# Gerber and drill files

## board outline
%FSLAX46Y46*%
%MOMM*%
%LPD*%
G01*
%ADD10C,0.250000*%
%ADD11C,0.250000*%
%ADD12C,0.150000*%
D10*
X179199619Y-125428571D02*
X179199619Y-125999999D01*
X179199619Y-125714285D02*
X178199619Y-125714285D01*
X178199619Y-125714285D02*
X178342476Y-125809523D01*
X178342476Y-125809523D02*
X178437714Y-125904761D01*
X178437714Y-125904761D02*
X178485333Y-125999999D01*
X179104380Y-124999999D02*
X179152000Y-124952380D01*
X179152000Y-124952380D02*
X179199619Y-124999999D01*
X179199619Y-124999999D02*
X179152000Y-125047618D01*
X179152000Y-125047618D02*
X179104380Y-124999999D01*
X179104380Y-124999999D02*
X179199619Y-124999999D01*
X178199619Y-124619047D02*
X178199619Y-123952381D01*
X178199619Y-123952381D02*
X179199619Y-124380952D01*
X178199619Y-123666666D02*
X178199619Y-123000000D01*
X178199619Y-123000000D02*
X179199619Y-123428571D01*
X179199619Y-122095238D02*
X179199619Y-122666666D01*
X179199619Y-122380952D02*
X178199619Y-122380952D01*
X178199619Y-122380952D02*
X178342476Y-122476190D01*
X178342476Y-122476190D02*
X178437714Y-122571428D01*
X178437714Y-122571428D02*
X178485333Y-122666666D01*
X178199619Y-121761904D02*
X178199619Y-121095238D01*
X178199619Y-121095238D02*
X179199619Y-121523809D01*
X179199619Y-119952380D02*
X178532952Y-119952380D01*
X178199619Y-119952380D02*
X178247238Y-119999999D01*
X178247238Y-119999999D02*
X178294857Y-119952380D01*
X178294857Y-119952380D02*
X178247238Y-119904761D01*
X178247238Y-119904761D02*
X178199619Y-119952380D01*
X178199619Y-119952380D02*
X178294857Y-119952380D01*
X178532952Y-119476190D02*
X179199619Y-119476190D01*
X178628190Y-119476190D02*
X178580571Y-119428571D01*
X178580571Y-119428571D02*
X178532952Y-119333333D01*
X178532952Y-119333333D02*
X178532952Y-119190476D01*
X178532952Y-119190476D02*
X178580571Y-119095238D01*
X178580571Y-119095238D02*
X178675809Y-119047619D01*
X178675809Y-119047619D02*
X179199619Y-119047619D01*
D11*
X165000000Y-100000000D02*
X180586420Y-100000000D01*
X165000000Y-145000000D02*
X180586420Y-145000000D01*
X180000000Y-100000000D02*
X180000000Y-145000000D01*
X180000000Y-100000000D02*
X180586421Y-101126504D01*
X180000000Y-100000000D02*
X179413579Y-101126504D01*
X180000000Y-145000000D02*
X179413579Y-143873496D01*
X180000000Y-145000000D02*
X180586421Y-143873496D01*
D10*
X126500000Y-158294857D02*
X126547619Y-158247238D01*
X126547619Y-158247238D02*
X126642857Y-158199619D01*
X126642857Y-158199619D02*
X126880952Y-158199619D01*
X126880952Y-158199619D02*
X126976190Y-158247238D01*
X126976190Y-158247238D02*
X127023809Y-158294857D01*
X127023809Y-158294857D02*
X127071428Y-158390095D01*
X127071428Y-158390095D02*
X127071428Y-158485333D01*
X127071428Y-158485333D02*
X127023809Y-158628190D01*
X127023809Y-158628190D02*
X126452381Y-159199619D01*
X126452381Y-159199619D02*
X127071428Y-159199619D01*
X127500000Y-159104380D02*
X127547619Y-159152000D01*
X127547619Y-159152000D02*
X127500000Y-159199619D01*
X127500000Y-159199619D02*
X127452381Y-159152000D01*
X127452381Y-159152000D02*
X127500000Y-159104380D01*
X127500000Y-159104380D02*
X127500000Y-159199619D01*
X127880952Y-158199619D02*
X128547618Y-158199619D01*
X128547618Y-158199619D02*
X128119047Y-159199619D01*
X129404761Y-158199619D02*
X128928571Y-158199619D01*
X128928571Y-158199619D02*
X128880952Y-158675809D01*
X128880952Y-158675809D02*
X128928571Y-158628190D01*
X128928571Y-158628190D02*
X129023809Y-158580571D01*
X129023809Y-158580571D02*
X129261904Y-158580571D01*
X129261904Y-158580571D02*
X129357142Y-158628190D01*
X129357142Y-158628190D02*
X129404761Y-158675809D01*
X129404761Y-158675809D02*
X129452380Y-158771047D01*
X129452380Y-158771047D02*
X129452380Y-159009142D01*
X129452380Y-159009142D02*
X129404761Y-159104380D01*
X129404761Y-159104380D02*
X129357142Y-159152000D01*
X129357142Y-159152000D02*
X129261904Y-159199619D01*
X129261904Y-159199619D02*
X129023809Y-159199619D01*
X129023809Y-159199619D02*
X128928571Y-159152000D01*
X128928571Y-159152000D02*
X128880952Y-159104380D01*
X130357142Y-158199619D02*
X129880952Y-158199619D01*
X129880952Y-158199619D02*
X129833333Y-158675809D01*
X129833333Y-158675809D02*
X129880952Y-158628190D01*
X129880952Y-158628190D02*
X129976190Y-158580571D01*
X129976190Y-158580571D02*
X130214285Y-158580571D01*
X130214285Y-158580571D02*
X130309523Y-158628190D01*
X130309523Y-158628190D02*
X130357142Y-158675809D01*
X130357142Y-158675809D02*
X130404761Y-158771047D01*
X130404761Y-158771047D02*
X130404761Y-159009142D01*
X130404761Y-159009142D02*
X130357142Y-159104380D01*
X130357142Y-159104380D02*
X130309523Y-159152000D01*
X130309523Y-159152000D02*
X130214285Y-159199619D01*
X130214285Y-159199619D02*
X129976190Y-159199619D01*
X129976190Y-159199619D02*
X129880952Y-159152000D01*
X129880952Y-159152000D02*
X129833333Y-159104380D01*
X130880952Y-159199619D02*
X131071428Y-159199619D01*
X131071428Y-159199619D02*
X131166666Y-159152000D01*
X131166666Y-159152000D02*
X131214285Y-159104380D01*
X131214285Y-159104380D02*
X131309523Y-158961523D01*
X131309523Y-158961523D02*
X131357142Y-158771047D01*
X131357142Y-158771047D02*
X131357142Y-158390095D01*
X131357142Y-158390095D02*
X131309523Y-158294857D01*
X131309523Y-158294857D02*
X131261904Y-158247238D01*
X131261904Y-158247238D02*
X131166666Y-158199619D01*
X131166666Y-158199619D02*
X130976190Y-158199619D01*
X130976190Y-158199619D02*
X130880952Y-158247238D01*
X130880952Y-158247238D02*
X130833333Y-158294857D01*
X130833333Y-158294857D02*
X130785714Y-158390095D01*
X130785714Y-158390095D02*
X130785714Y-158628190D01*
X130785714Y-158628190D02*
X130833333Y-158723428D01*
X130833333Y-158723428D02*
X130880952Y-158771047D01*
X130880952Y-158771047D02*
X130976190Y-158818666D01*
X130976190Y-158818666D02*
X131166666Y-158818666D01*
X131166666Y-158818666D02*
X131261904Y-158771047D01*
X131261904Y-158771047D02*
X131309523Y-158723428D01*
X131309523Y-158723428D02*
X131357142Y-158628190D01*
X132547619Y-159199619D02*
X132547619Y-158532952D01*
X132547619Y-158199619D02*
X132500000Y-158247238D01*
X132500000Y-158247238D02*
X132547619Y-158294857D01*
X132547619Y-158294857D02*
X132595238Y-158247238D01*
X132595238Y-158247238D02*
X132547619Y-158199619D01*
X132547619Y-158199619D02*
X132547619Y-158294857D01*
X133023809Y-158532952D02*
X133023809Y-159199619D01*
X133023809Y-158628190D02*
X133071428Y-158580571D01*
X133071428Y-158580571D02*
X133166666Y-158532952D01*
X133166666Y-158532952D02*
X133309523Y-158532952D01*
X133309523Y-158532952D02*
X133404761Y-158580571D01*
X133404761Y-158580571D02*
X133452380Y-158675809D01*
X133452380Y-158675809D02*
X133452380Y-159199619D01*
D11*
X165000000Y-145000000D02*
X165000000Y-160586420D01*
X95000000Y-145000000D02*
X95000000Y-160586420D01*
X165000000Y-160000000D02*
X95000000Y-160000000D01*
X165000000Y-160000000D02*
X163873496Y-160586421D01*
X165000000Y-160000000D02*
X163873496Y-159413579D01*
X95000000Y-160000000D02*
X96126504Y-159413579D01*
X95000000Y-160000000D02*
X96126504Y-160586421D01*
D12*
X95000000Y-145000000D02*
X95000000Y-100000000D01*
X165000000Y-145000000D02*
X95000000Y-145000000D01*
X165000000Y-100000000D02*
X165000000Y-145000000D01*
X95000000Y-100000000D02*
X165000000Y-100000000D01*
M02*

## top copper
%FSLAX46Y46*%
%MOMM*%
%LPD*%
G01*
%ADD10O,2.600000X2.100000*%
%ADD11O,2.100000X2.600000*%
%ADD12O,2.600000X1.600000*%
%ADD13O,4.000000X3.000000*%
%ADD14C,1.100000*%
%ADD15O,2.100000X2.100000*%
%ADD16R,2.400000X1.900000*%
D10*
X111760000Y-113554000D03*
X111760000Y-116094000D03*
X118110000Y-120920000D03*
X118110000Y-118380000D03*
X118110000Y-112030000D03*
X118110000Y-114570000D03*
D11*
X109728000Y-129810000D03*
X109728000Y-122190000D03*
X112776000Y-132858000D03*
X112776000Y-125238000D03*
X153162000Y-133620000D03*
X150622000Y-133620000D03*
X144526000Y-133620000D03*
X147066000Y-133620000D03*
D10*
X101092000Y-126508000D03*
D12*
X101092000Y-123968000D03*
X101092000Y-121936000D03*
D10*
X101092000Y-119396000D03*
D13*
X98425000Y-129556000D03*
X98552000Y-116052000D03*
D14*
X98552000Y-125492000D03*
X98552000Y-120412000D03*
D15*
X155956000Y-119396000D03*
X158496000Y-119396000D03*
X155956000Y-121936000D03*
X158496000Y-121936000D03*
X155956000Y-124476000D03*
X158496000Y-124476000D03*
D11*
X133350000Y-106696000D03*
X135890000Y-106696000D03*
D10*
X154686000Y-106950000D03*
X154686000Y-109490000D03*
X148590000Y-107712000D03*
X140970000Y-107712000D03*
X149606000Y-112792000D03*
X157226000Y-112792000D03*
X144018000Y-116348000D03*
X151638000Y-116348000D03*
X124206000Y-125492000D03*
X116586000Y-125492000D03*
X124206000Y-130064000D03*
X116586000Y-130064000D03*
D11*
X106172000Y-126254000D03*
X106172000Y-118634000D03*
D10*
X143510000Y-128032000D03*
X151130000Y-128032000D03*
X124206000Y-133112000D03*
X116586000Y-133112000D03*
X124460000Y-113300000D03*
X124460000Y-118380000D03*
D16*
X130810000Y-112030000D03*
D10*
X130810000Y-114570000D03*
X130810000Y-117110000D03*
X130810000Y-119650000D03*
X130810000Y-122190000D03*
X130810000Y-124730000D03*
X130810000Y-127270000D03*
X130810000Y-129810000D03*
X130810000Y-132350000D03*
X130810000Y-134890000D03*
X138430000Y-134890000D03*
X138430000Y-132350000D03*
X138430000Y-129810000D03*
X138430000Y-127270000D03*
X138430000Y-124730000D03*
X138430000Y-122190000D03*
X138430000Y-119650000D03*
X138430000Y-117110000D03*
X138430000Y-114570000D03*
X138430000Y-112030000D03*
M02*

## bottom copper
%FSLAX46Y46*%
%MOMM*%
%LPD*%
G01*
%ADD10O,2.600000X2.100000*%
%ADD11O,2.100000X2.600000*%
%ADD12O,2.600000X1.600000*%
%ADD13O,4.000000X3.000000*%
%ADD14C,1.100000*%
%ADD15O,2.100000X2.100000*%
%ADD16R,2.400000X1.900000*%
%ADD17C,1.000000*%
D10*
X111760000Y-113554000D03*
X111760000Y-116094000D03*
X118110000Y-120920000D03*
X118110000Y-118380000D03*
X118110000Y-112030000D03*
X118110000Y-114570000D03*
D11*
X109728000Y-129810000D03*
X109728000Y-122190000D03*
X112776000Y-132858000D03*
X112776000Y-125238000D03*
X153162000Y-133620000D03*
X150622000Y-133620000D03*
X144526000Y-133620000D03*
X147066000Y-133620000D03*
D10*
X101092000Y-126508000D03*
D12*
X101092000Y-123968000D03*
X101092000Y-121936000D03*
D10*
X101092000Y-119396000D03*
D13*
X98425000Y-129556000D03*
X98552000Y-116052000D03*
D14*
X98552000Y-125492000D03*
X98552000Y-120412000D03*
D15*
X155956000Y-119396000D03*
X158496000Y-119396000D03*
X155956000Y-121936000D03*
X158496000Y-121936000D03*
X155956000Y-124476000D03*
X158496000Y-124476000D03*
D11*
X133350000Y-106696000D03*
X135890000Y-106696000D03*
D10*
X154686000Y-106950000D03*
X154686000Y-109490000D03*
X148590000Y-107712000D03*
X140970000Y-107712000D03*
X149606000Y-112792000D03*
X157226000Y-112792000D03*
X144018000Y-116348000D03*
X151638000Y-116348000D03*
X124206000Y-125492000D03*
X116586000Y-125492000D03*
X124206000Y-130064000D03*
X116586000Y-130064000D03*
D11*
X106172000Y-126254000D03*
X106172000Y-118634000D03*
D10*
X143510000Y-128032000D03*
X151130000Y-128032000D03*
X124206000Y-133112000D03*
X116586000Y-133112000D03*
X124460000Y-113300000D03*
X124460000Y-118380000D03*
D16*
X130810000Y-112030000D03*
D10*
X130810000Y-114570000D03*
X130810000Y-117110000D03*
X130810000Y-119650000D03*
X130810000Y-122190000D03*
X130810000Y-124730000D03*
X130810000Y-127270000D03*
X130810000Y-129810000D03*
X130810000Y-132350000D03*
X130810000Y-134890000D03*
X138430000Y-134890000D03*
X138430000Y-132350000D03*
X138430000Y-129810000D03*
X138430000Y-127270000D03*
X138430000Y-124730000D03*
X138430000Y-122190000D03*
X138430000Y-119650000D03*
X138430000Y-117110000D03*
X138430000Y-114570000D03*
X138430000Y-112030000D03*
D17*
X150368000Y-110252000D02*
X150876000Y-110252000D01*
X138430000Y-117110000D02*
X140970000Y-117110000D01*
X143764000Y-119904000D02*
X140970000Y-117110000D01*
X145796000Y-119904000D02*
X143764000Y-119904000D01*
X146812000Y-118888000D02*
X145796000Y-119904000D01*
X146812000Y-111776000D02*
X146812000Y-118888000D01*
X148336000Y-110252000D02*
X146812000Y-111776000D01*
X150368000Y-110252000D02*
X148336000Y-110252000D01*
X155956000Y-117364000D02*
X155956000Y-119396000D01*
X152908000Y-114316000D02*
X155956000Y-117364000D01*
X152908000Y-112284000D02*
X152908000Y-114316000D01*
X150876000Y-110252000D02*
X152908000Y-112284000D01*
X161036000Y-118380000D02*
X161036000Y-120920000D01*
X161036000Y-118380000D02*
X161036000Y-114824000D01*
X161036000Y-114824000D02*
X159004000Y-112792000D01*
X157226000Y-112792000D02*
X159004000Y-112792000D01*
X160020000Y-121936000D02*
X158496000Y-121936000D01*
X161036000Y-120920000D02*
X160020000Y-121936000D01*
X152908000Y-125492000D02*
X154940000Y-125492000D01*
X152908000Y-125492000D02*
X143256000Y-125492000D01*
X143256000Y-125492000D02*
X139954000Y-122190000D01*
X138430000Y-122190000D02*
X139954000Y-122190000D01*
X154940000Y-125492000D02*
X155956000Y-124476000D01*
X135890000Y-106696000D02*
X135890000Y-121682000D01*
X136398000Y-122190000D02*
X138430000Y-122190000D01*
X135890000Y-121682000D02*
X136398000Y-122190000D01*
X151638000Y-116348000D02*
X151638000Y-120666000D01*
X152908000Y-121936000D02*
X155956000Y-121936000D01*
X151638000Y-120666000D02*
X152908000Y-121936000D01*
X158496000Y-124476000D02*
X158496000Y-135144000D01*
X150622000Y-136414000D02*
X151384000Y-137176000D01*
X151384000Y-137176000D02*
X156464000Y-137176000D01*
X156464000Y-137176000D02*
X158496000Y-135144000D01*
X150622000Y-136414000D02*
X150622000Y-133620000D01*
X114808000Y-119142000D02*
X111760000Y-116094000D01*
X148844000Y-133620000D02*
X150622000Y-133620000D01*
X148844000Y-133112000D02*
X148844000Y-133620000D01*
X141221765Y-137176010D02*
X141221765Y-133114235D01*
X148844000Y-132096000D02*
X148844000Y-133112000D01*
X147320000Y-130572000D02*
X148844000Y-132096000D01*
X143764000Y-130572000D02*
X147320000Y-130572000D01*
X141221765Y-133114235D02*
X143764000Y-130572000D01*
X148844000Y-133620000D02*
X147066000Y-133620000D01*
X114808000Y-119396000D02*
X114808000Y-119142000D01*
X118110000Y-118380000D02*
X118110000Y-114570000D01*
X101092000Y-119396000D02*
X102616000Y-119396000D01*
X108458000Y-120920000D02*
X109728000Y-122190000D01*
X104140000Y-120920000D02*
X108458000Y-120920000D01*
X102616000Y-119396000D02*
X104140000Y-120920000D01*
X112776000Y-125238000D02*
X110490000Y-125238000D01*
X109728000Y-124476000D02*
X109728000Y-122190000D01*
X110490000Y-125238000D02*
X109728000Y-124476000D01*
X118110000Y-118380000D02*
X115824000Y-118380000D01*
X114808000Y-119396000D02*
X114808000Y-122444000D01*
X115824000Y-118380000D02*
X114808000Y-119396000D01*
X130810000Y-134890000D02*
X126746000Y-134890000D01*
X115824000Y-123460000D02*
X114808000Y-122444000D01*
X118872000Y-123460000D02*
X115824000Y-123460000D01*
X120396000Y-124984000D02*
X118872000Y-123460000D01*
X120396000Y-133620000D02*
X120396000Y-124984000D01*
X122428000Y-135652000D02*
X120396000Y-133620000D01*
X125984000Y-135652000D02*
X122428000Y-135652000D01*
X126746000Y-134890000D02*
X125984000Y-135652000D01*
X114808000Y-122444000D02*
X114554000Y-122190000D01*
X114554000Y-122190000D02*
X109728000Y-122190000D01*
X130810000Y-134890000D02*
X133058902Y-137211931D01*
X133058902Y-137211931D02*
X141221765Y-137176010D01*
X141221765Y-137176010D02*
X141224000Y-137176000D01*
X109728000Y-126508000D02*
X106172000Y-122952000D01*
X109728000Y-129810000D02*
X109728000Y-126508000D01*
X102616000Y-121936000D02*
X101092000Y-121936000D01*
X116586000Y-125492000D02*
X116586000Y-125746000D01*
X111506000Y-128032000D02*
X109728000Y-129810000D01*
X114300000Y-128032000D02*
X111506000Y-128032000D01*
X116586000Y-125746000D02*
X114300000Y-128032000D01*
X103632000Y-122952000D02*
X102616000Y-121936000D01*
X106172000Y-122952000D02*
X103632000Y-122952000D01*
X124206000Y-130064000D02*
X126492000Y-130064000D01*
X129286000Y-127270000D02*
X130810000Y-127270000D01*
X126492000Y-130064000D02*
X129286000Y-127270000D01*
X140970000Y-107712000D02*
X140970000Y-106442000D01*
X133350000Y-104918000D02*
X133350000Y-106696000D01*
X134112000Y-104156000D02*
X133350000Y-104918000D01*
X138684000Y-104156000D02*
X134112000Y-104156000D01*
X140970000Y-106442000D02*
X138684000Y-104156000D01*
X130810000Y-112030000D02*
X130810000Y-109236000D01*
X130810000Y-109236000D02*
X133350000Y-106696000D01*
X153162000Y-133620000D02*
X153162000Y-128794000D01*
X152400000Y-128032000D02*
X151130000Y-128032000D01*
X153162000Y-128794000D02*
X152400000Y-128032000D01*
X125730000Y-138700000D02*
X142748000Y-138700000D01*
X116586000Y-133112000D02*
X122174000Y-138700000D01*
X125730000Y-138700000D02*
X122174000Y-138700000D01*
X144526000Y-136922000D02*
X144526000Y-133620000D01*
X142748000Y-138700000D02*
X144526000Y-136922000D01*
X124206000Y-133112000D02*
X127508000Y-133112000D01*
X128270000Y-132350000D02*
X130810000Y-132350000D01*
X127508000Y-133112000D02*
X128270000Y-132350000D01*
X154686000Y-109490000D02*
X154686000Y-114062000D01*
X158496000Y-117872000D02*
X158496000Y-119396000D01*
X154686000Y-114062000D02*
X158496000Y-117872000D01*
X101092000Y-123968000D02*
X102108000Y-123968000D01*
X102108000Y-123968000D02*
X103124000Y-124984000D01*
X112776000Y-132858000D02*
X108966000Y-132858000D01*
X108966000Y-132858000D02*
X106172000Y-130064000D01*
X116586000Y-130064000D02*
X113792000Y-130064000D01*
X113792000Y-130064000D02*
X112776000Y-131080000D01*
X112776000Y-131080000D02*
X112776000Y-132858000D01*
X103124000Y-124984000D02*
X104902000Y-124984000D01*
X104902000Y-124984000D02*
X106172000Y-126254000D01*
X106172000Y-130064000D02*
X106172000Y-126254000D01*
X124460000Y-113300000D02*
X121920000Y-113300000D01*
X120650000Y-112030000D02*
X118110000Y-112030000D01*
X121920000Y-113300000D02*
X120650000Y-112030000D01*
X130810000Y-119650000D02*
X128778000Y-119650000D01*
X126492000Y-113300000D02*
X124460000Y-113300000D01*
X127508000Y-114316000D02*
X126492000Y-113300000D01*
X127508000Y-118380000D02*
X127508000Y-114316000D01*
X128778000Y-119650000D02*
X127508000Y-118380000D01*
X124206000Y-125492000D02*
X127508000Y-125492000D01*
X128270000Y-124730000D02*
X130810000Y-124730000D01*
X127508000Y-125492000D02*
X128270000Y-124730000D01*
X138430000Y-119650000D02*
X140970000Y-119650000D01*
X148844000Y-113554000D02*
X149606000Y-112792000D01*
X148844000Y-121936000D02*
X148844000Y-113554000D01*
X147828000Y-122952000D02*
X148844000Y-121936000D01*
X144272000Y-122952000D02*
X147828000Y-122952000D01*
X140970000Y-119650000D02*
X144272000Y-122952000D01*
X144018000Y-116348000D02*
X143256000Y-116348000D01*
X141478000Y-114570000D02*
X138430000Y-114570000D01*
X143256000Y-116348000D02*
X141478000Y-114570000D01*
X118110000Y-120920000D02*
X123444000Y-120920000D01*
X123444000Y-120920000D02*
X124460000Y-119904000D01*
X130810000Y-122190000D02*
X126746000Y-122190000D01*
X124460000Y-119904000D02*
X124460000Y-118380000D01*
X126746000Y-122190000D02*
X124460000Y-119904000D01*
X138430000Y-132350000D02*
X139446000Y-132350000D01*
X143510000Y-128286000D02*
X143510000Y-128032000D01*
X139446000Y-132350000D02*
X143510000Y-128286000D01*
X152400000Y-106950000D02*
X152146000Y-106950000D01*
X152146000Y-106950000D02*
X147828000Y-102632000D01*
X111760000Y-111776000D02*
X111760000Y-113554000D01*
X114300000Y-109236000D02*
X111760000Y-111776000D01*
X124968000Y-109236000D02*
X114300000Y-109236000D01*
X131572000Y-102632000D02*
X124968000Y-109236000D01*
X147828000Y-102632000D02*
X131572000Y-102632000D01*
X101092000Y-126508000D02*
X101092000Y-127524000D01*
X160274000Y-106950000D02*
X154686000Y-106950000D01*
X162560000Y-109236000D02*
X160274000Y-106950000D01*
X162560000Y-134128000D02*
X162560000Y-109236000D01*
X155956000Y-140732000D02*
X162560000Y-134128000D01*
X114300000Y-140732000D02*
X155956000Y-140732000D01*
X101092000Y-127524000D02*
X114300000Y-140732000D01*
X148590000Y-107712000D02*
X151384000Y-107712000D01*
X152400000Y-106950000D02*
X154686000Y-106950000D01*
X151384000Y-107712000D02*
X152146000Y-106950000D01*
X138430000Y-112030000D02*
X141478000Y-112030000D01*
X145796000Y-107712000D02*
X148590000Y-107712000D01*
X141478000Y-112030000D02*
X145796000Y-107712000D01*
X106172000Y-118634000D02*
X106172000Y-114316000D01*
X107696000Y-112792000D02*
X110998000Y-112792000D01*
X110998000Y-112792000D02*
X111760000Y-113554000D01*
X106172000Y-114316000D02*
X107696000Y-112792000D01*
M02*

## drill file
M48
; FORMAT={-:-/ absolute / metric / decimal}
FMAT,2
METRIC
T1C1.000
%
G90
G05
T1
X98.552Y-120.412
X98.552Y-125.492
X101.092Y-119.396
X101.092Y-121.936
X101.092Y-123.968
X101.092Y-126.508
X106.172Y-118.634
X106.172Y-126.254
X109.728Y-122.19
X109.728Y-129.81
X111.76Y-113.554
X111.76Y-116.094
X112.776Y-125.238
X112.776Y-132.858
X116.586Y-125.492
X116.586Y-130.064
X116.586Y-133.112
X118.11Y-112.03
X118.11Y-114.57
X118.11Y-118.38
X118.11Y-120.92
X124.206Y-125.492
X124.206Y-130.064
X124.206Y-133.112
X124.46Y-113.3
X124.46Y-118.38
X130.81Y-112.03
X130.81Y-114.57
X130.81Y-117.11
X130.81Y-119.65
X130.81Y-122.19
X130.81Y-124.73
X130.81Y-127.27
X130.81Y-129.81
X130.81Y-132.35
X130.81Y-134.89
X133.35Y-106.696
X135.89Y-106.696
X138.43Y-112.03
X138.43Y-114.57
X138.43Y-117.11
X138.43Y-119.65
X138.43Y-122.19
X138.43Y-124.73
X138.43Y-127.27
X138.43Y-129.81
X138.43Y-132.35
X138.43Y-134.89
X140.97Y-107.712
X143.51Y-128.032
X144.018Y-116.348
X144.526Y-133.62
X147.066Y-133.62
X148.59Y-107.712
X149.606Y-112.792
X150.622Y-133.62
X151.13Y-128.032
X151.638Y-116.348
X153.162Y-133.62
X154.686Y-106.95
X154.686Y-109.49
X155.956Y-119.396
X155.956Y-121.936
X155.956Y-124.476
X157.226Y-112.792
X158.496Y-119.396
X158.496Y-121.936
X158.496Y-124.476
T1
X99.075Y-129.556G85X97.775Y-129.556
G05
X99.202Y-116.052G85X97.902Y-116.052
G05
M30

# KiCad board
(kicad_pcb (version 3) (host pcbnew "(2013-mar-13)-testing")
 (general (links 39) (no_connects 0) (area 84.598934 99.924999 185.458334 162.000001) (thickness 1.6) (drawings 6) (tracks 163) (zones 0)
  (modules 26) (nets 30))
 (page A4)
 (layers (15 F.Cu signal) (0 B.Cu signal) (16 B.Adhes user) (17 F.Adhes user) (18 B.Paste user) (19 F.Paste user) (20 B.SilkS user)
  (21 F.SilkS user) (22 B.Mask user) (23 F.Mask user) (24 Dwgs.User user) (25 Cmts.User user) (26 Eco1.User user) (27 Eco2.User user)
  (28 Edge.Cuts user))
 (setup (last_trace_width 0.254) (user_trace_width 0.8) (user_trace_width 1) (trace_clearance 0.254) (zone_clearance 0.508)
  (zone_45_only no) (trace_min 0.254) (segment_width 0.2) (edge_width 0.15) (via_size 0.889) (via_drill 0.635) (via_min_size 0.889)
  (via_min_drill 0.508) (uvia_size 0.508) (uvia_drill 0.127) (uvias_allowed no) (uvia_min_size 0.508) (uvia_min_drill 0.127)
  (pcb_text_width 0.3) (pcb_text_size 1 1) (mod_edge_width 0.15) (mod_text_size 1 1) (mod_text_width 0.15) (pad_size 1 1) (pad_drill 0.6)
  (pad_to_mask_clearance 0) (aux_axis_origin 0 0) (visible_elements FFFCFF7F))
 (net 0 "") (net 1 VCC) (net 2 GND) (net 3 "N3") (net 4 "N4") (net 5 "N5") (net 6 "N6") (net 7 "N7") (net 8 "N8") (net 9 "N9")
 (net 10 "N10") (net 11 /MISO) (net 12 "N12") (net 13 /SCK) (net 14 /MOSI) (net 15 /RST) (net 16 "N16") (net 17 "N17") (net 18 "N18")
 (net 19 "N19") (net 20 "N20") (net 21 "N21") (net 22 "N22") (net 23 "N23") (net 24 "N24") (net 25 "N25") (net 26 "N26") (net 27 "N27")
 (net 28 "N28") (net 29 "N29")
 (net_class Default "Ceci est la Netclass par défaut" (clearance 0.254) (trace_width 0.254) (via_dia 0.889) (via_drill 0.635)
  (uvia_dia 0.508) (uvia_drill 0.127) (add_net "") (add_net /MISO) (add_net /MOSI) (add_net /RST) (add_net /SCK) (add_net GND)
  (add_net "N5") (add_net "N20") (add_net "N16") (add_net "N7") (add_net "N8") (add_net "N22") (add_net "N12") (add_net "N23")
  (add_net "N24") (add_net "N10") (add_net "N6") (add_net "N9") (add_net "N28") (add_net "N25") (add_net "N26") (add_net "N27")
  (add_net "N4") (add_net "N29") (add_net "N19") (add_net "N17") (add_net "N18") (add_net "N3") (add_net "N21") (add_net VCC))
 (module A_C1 (layer F.Cu) (at 111.76 114.824 270)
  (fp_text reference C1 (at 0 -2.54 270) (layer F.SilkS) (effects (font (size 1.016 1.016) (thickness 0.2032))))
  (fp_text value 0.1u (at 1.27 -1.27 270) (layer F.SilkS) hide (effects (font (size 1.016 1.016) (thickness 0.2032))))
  (pad 1 thru_hole oval (at -1.27 0 270) (size 2.1 2.6) (drill 1) (layers *.Cu *.Mask F.SilkS) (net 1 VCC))
  (pad 2 thru_hole oval (at 1.27 0 270) (size 2.1 2.6) (drill 1) (layers *.Cu *.Mask F.SilkS) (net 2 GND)))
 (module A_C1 (layer F.Cu) (at 118.11 119.65 90)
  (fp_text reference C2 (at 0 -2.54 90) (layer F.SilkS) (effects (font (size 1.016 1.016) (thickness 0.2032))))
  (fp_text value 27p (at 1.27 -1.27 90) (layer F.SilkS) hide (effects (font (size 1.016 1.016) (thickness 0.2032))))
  (pad 1 thru_hole oval (at -1.27 0 90) (size 2.1 2.6) (drill 1) (layers *.Cu *.Mask F.SilkS) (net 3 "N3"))
  (pad 2 thru_hole oval (at 1.27 0 90) (size 2.1 2.6) (drill 1) (layers *.Cu *.Mask F.SilkS) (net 2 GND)))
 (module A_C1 (layer F.Cu) (at 118.11 113.3 270)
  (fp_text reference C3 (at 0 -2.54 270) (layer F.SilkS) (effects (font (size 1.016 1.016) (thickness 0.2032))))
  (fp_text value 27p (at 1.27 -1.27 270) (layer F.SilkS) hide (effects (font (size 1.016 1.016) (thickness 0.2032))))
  (pad 1 thru_hole oval (at -1.27 0 270) (size 2.1 2.6) (drill 1) (layers *.Cu *.Mask F.SilkS) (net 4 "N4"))
  (pad 2 thru_hole oval (at 1.27 0 270) (size 2.1 2.6) (drill 1) (layers *.Cu *.Mask F.SilkS) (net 2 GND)))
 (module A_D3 (layer F.Cu) (at 109.728 126 270)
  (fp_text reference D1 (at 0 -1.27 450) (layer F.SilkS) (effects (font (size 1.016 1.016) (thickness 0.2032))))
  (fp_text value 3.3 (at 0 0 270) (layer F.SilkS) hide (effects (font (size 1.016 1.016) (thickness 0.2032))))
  (pad 2 thru_hole oval (at 3.81 0 270) (size 2.6 2.1) (drill 1) (layers *.Cu *.Mask F.SilkS) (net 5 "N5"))
  (pad 1 thru_hole oval (at -3.81 0 270) (size 2.6 2.1) (drill 1) (layers *.Cu *.Mask F.SilkS) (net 2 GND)))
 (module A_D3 (layer F.Cu) (at 112.776 129.048 270)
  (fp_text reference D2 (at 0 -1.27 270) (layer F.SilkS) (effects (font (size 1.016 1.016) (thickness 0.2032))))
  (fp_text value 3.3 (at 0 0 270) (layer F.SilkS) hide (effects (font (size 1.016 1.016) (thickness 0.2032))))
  (pad 2 thru_hole oval (at 3.81 0 270) (size 2.6 2.1) (drill 1) (layers *.Cu *.Mask F.SilkS) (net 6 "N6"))
  (pad 1 thru_hole oval (at -3.81 0 270) (size 2.6 2.1) (drill 1) (layers *.Cu *.Mask F.SilkS) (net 2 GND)))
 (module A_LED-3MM (layer F.Cu) (at 151.892 133.62 180)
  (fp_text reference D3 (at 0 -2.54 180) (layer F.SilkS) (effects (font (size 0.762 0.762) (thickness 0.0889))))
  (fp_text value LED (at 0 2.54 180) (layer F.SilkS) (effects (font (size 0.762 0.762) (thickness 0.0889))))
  (pad 1 thru_hole oval (at -1.27 0 180) (size 2.1 2.6) (drill 1) (layers *.Cu *.Mask F.SilkS) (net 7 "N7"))
  (pad 2 thru_hole oval (at 1.27 0 180) (size 2.1 2.6) (drill 1) (layers *.Cu *.Mask F.SilkS) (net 2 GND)))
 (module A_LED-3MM (layer F.Cu) (at 145.796 133.62)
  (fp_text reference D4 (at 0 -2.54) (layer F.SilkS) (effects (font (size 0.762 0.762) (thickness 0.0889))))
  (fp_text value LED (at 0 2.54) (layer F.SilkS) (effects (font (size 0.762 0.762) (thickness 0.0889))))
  (pad 1 thru_hole oval (at -1.27 0) (size 2.1 2.6) (drill 1) (layers *.Cu *.Mask F.SilkS) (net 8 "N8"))
  (pad 2 thru_hole oval (at 1.27 0) (size 2.1 2.6) (drill 1) (layers *.Cu *.Mask F.SilkS) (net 2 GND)))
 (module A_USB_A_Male (layer F.Cu) (at 101.092 122.952 180)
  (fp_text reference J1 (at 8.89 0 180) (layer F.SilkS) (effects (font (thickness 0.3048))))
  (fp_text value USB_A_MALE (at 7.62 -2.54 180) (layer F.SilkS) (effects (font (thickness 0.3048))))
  (pad 1 thru_hole oval (at 0 -3.556 180) (size 2.6 2.1) (drill 1) (layers *.Cu *.Mask F.SilkS) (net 1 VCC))
  (pad 2 thru_hole oval (at 0 -1.016 180) (size 2.6 1.6) (drill 1) (layers *.Cu *.Mask F.SilkS) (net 6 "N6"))
  (pad 3 thru_hole oval (at 0 1.016 180) (size 2.6 1.6) (drill 1) (layers *.Cu *.Mask F.SilkS) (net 5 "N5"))
  (pad 4 thru_hole oval (at 0 3.556 180) (size 2.6 2.1) (drill 1) (layers *.Cu *.Mask F.SilkS) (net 2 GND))
  (pad 6 thru_hole oval (at 2.667 -6.604 180) (size 4 3) (drill oval 2.3 1) (layers *.Cu *.Mask F.SilkS) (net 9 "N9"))
  (pad 5 thru_hole oval (at 2.54 6.9 180) (size 4 3) (drill oval 2.3 1) (layers *.Cu *.Mask F.SilkS) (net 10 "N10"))
  (pad "" thru_hole circle (at 2.54 -2.54 180) (size 1.1 1.1) (drill 1) (layers *.Cu *.Mask F.SilkS))
  (pad "" thru_hole circle (at 2.54 2.54 180) (size 1.1 1.1) (drill 1) (layers *.Cu *.Mask F.SilkS)))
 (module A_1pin (layer F.Cu) (at 155.956 119.396)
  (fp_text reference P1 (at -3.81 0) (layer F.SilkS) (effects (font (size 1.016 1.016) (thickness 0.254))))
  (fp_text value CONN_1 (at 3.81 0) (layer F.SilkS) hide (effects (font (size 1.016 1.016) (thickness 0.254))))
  (pad 1 thru_hole oval (at 0 0) (size 2.1 2.1) (drill 1) (layers *.Cu *.Mask F.SilkS) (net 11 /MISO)))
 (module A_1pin (layer F.Cu) (at 158.496 119.396)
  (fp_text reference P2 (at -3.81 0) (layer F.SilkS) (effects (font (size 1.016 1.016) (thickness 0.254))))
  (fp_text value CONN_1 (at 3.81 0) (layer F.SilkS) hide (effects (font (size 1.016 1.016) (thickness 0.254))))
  (pad 1 thru_hole oval (at 0 0) (size 2.1 2.1) (drill 1) (layers *.Cu *.Mask F.SilkS) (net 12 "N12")))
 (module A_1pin (layer F.Cu) (at 155.956 121.936)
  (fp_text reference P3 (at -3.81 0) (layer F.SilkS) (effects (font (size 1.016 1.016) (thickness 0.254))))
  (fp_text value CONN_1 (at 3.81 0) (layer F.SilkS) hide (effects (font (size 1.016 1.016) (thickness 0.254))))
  (pad 1 thru_hole oval (at 0 0) (size 2.1 2.1) (drill 1) (layers *.Cu *.Mask F.SilkS) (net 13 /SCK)))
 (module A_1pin (layer F.Cu) (at 158.496 121.936)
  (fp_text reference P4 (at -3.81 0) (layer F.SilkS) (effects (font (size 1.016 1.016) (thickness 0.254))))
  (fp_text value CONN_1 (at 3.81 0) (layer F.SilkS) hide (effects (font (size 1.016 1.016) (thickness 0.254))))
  (pad 1 thru_hole oval (at 0 0) (size 2.1 2.1) (drill 1) (layers *.Cu *.Mask F.SilkS) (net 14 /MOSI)))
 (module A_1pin (layer F.Cu) (at 155.956 124.476)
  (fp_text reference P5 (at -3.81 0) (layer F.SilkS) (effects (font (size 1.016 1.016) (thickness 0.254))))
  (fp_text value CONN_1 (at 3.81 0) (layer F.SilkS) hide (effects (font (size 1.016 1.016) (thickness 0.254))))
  (pad 1 thru_hole oval (at 0 0) (size 2.1 2.1) (drill 1) (layers *.Cu *.Mask F.SilkS) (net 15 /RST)))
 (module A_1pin (layer F.Cu) (at 158.496 124.476)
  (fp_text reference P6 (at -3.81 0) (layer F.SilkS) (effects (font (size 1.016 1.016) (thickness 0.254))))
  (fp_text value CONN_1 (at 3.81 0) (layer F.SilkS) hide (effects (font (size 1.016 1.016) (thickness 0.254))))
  (pad 1 thru_hole oval (at 0 0) (size 2.1 2.1) (drill 1) (layers *.Cu *.Mask F.SilkS) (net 2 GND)))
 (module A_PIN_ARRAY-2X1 (layer F.Cu) (at 134.62 106.696)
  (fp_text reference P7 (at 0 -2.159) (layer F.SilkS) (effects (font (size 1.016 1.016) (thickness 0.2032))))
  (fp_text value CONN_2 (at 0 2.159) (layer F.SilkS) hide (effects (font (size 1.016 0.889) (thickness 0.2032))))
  (pad 1 thru_hole oval (at -1.27 0) (size 2.1 2.6) (drill 1) (layers *.Cu *.Mask F.SilkS) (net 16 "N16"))
  (pad 2 thru_hole oval (at 1.27 0) (size 2.1 2.6) (drill 1) (layers *.Cu *.Mask F.SilkS) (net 15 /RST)))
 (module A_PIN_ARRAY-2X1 (layer F.Cu) (at 154.686 108.22 270)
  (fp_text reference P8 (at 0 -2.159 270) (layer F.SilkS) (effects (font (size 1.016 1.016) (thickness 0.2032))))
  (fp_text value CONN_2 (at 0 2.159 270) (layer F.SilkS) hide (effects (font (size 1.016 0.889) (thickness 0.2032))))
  (pad 1 thru_hole oval (at -1.27 0 270) (size 2.1 2.6) (drill 1) (layers *.Cu *.Mask F.SilkS) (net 1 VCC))
  (pad 2 thru_hole oval (at 1.27 0 270) (size 2.1 2.6) (drill 1) (layers *.Cu *.Mask F.SilkS) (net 12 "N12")))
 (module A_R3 (layer F.Cu) (at 144.78 107.712 180) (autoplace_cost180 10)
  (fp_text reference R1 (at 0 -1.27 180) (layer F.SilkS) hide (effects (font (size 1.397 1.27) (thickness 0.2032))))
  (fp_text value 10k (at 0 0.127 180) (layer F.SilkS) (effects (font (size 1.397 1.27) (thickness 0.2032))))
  (pad 1 thru_hole oval (at -3.81 0 180) (size 2.6 2.1) (drill 1) (layers *.Cu *.Mask F.SilkS) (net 1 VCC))
  (pad 2 thru_hole oval (at 3.81 0 180) (size 2.6 2.1) (drill 1) (layers *.Cu *.Mask F.SilkS) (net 16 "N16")))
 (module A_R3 (layer F.Cu) (at 153.416 112.792) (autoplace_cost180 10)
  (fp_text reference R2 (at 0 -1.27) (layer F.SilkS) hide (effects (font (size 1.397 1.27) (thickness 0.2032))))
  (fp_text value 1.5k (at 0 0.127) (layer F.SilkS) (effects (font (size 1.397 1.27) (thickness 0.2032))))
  (pad 1 thru_hole oval (at -3.81 0) (size 2.6 2.1) (drill 1) (layers *.Cu *.Mask F.SilkS) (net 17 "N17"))
  (pad 2 thru_hole oval (at 3.81 0) (size 2.6 2.1) (drill 1) (layers *.Cu *.Mask F.SilkS) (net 14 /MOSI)))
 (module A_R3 (layer F.Cu) (at 147.828 116.348) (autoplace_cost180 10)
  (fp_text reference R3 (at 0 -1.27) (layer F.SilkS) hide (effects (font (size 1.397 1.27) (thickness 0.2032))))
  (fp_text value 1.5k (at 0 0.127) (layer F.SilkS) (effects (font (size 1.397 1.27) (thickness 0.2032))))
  (pad 1 thru_hole oval (at -3.81 0) (size 2.6 2.1) (drill 1) (layers *.Cu *.Mask F.SilkS) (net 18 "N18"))
  (pad 2 thru_hole oval (at 3.81 0) (size 2.6 2.1) (drill 1) (layers *.Cu *.Mask F.SilkS) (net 13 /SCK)))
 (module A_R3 (layer F.Cu) (at 120.396 125.492 180) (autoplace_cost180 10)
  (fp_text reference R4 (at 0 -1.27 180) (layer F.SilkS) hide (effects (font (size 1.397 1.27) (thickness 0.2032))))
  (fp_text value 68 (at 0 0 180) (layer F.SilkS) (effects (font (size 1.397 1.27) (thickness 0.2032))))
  (pad 1 thru_hole oval (at -3.81 0 180) (size 2.6 2.1) (drill 1) (layers *.Cu *.Mask F.SilkS) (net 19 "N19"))
  (pad 2 thru_hole oval (at 3.81 0 180) (size 2.6 2.1) (drill 1) (layers *.Cu *.Mask F.SilkS) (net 5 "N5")))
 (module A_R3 (layer F.Cu) (at 120.396 130.064 180) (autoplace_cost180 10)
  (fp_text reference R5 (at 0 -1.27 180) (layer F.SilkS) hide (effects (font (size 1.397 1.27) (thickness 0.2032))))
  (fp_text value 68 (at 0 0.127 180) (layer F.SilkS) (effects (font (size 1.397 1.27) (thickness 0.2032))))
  (pad 1 thru_hole oval (at -3.81 0 180) (size 2.6 2.1) (drill 1) (layers *.Cu *.Mask F.SilkS) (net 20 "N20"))
  (pad 2 thru_hole oval (at 3.81 0 180) (size 2.6 2.1) (drill 1) (layers *.Cu *.Mask F.SilkS) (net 6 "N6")))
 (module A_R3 (layer F.Cu) (at 106.172 122.444 90) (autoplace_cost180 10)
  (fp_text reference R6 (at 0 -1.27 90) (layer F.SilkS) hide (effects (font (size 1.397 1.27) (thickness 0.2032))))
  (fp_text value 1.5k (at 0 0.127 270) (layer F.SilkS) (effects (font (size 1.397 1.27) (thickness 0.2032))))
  (pad 1 thru_hole oval (at -3.81 0 90) (size 2.6 2.1) (drill 1) (layers *.Cu *.Mask F.SilkS) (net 6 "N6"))
  (pad 2 thru_hole oval (at 3.81 0 90) (size 2.6 2.1) (drill 1) (layers *.Cu *.Mask F.SilkS) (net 1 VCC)))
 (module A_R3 (layer F.Cu) (at 147.32 128.032) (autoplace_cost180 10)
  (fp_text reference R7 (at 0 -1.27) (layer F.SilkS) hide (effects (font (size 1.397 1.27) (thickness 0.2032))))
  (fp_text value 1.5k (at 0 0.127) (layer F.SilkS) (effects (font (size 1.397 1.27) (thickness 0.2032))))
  (pad 1 thru_hole oval (at -3.81 0) (size 2.6 2.1) (drill 1) (layers *.Cu *.Mask F.SilkS) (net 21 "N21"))
  (pad 2 thru_hole oval (at 3.81 0) (size 2.6 2.1) (drill 1) (layers *.Cu *.Mask F.SilkS) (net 7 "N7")))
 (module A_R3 (layer F.Cu) (at 120.396 133.112 180) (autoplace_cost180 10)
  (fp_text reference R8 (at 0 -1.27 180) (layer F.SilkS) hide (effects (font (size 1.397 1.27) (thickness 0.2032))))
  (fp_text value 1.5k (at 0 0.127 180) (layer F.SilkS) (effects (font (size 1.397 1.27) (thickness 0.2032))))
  (pad 1 thru_hole oval (at -3.81 0 180) (size 2.6 2.1) (drill 1) (layers *.Cu *.Mask F.SilkS) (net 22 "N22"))
  (pad 2 thru_hole oval (at 3.81 0 180) (size 2.6 2.1) (drill 1) (layers *.Cu *.Mask F.SilkS) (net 8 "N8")))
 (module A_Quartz (layer F.Cu) (at 124.46 114.57 270)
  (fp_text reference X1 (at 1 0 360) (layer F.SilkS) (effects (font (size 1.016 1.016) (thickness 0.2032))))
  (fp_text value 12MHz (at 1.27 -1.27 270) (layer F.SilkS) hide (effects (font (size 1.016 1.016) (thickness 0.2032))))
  (pad 1 thru_hole oval (at -1.27 0 270) (size 2.1 2.6) (drill 1) (layers *.Cu *.Mask F.SilkS) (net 4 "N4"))
  (pad 2 thru_hole oval (at 3.81 0 270) (size 2.1 2.6) (drill 1) (layers *.Cu *.Mask F.SilkS) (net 3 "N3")))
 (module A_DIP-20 (layer F.Cu) (at 134.62 123.46 270)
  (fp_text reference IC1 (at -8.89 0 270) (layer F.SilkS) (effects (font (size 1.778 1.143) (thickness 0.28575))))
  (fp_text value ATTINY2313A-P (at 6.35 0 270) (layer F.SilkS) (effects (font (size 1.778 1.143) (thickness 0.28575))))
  (pad 1 thru_hole rect (at -11.43 3.81 270) (size 1.9 2.4) (drill 1) (layers *.Cu *.Mask F.SilkS) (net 16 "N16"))
  (pad 2 thru_hole oval (at -8.89 3.81 270) (size 2.1 2.6) (drill 1) (layers *.Cu *.Mask F.SilkS) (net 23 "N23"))
  (pad 3 thru_hole oval (at -6.35 3.81 270) (size 2.1 2.6) (drill 1) (layers *.Cu *.Mask F.SilkS) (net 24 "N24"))
  (pad 4 thru_hole oval (at -3.81 3.81 270) (size 2.1 2.6) (drill 1) (layers *.Cu *.Mask F.SilkS) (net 4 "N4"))
  (pad 5 thru_hole oval (at -1.27 3.81 270) (size 2.1 2.6) (drill 1) (layers *.Cu *.Mask F.SilkS) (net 3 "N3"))
  (pad 6 thru_hole oval (at 1.27 3.81 270) (size 2.1 2.6) (drill 1) (layers *.Cu *.Mask F.SilkS) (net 19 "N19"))
  (pad 7 thru_hole oval (at 3.81 3.81 270) (size 2.1 2.6) (drill 1) (layers *.Cu *.Mask F.SilkS) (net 20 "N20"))
  (pad 8 thru_hole oval (at 6.35 3.81 270) (size 2.1 2.6) (drill 1) (layers *.Cu *.Mask F.SilkS) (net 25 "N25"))
  (pad 9 thru_hole oval (at 8.89 3.81 270) (size 2.1 2.6) (drill 1) (layers *.Cu *.Mask F.SilkS) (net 22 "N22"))
  (pad 10 thru_hole oval (at 11.43 3.81 270) (size 2.1 2.6) (drill 1) (layers *.Cu *.Mask F.SilkS) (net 2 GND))
  (pad 11 thru_hole oval (at 11.43 -3.81 270) (size 2.1 2.6) (drill 1) (layers *.Cu *.Mask F.SilkS) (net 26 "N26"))
  (pad 12 thru_hole oval (at 8.89 -3.81 270) (size 2.1 2.6) (drill 1) (layers *.Cu *.Mask F.SilkS) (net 21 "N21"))
  (pad 13 thru_hole oval (at 6.35 -3.81 270) (size 2.1 2.6) (drill 1) (layers *.Cu *.Mask F.SilkS) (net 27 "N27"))
  (pad 14 thru_hole oval (at 3.81 -3.81 270) (size 2.1 2.6) (drill 1) (layers *.Cu *.Mask F.SilkS) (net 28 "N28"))
  (pad 15 thru_hole oval (at 1.27 -3.81 270) (size 2.1 2.6) (drill 1) (layers *.Cu *.Mask F.SilkS) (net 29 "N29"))
  (pad 16 thru_hole oval (at -1.27 -3.81 270) (size 2.1 2.6) (drill 1) (layers *.Cu *.Mask F.SilkS) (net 15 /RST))
  (pad 17 thru_hole oval (at -3.81 -3.81 270) (size 2.1 2.6) (drill 1) (layers *.Cu *.Mask F.SilkS) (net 17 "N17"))
  (pad 18 thru_hole oval (at -6.35 -3.81 270) (size 2.1 2.6) (drill 1) (layers *.Cu *.Mask F.SilkS) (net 11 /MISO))
  (pad 19 thru_hole oval (at -8.89 -3.81 270) (size 2.1 2.6) (drill 1) (layers *.Cu *.Mask F.SilkS) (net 18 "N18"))
  (pad 20 thru_hole oval (at -11.43 -3.81 270) (size 2.1 2.6) (drill 1) (layers *.Cu *.Mask F.SilkS) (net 1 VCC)))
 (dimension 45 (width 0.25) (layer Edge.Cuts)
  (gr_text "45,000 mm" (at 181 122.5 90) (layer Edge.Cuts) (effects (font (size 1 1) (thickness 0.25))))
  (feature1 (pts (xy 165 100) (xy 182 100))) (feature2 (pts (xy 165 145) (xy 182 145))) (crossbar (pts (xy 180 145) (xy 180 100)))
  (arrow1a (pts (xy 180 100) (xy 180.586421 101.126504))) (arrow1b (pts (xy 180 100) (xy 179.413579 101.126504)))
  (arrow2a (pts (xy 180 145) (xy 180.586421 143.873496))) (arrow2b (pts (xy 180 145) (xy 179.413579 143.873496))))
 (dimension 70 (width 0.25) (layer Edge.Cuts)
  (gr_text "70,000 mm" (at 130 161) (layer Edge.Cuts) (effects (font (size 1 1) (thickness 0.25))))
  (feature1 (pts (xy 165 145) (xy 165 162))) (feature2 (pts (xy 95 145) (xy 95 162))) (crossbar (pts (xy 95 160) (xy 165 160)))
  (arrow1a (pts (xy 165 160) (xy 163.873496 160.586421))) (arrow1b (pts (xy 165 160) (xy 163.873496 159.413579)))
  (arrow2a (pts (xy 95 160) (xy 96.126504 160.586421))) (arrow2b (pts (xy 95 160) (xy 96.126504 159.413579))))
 (gr_line (start 95 145) (end 95 100) (angle 90) (layer Edge.Cuts) (width 0.15))
 (gr_line (start 165 145) (end 95 145) (angle 90) (layer Edge.Cuts) (width 0.15))
 (gr_line (start 165 100) (end 165 145) (angle 90) (layer Edge.Cuts) (width 0.15))
 (gr_line (start 95 100) (end 165 100) (angle 90) (layer Edge.Cuts) (width 0.15))
 (segment (start 150.368 110.252) (end 150.876 110.252) (width 1) (layer B.Cu) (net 11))
 (segment (start 138.43 117.11) (end 140.97 117.11) (width 1) (layer B.Cu) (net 11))
 (segment (start 143.764 119.904) (end 140.97 117.11) (width 1) (layer B.Cu) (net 11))
 (segment (start 145.796 119.904) (end 143.764 119.904) (width 1) (layer B.Cu) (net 11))
 (segment (start 146.812 118.888) (end 145.796 119.904) (width 1) (layer B.Cu) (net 11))
 (segment (start 146.812 111.776) (end 146.812 118.888) (width 1) (layer B.Cu) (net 11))
 (segment (start 148.336 110.252) (end 146.812 111.776) (width 1) (layer B.Cu) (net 11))
 (segment (start 150.368 110.252) (end 148.336 110.252) (width 1) (layer B.Cu) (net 11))
 (segment (start 155.956 117.364) (end 155.956 119.396) (width 1) (layer B.Cu) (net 11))
 (segment (start 152.908 114.316) (end 155.956 117.364) (width 1) (layer B.Cu) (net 11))
 (segment (start 152.908 112.284) (end 152.908 114.316) (width 1) (layer B.Cu) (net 11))
 (segment (start 150.876 110.252) (end 152.908 112.284) (width 1) (layer B.Cu) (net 11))
 (segment (start 161.036 118.38) (end 161.036 120.92) (width 1) (layer B.Cu) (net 14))
 (segment (start 161.036 118.38) (end 161.036 114.824) (width 1) (layer B.Cu) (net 14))
 (segment (start 161.036 114.824) (end 159.004 112.792) (width 1) (layer B.Cu) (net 14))
 (segment (start 157.226 112.792) (end 159.004 112.792) (width 1) (layer B.Cu) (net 14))
 (segment (start 160.02 121.936) (end 158.496 121.936) (width 1) (layer B.Cu) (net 14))
 (segment (start 161.036 120.92) (end 160.02 121.936) (width 1) (layer B.Cu) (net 14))
 (segment (start 152.908 125.492) (end 154.94 125.492) (width 1) (layer B.Cu) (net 15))
 (segment (start 152.908 125.492) (end 143.256 125.492) (width 1) (layer B.Cu) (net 15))
 (segment (start 143.256 125.492) (end 139.954 122.19) (width 1) (layer B.Cu) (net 15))
 (segment (start 138.43 122.19) (end 139.954 122.19) (width 1) (layer B.Cu) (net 15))
 (segment (start 154.94 125.492) (end 155.956 124.476) (width 1) (layer B.Cu) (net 15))
 (segment (start 135.89 106.696) (end 135.89 121.682) (width 1) (layer B.Cu) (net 15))
 (segment (start 136.398 122.19) (end 138.43 122.19) (width 1) (layer B.Cu) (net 15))
 (segment (start 135.89 121.682) (end 136.398 122.19) (width 1) (layer B.Cu) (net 15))
 (segment (start 151.638 116.348) (end 151.638 120.666) (width 1) (layer B.Cu) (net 13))
 (segment (start 152.908 121.936) (end 155.956 121.936) (width 1) (layer B.Cu) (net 13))
 (segment (start 151.638 120.666) (end 152.908 121.936) (width 1) (layer B.Cu) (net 13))
 (segment (start 158.496 124.476) (end 158.496 135.144) (width 1) (layer B.Cu) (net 2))
 (segment (start 150.622 136.414) (end 151.384 137.176) (width 1) (layer B.Cu) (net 2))
 (segment (start 151.384 137.176) (end 156.464 137.176) (width 1) (layer B.Cu) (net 2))
 (segment (start 156.464 137.176) (end 158.496 135.144) (width 1) (layer B.Cu) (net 2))
 (segment (start 150.622 136.414) (end 150.622 133.62) (width 1) (layer B.Cu) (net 2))
 (segment (start 114.808 119.142) (end 111.76 116.094) (width 1) (layer B.Cu) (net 2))
 (segment (start 148.844 133.62) (end 150.622 133.62) (width 1) (layer B.Cu) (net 2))
 (segment (start 148.844 133.112) (end 148.844 133.62) (width 1) (layer B.Cu) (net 2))
 (segment (start 141.221765 137.17601) (end 141.221765 133.114235) (width 1) (layer B.Cu) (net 2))
 (segment (start 148.844 132.096) (end 148.844 133.112) (width 1) (layer B.Cu) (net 2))
 (segment (start 147.32 130.572) (end 148.844 132.096) (width 1) (layer B.Cu) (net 2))
 (segment (start 143.764 130.572) (end 147.32 130.572) (width 1) (layer B.Cu) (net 2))
 (segment (start 141.221765 133.114235) (end 143.764 130.572) (width 1) (layer B.Cu) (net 2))
 (segment (start 148.844 133.62) (end 147.066 133.62) (width 1) (layer B.Cu) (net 2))
 (segment (start 114.808 119.396) (end 114.808 119.142) (width 1) (layer B.Cu) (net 2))
 (segment (start 118.11 118.38) (end 118.11 114.57) (width 1) (layer B.Cu) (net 2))
 (segment (start 101.092 119.396) (end 102.616 119.396) (width 1) (layer B.Cu) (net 2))
 (segment (start 108.458 120.92) (end 109.728 122.19) (width 1) (layer B.Cu) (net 2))
 (segment (start 104.14 120.92) (end 108.458 120.92) (width 1) (layer B.Cu) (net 2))
 (segment (start 102.616 119.396) (end 104.14 120.92) (width 1) (layer B.Cu) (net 2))
 (segment (start 112.776 125.238) (end 110.49 125.238) (width 1) (layer B.Cu) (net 2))
 (segment (start 109.728 124.476) (end 109.728 122.19) (width 1) (layer B.Cu) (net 2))
 (segment (start 110.49 125.238) (end 109.728 124.476) (width 1) (layer B.Cu) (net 2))
 (segment (start 118.11 118.38) (end 115.824 118.38) (width 1) (layer B.Cu) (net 2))
 (segment (start 114.808 119.396) (end 114.808 122.444) (width 1) (layer B.Cu) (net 2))
 (segment (start 115.824 118.38) (end 114.808 119.396) (width 1) (layer B.Cu) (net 2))
 (segment (start 130.81 134.89) (end 126.746 134.89) (width 1) (layer B.Cu) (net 2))
 (segment (start 115.824 123.46) (end 114.808 122.444) (width 1) (layer B.Cu) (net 2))
 (segment (start 118.872 123.46) (end 115.824 123.46) (width 1) (layer B.Cu) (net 2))
 (segment (start 120.396 124.984) (end 118.872 123.46) (width 1) (layer B.Cu) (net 2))
 (segment (start 120.396 133.62) (end 120.396 124.984) (width 1) (layer B.Cu) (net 2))
 (segment (start 122.428 135.652) (end 120.396 133.62) (width 1) (layer B.Cu) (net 2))
 (segment (start 125.984 135.652) (end 122.428 135.652) (width 1) (layer B.Cu) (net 2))
 (segment (start 126.746 134.89) (end 125.984 135.652) (width 1) (layer B.Cu) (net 2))
 (segment (start 114.808 122.444) (end 114.554 122.19) (width 1) (layer B.Cu) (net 2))
 (segment (start 114.554 122.19) (end 109.728 122.19) (width 1) (layer B.Cu) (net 2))
 (segment (start 130.81 134.89) (end 133.058902 137.211931) (width 1) (layer B.Cu) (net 2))
 (segment (start 133.058902 137.211931) (end 141.221765 137.17601) (width 1) (layer B.Cu) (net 2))
 (segment (start 141.221765 137.17601) (end 141.224 137.176) (width 1) (layer B.Cu) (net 2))
 (segment (start 109.728 126.508) (end 106.172 122.952) (width 1) (layer B.Cu) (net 5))
 (segment (start 109.728 129.81) (end 109.728 126.508) (width 1) (layer B.Cu) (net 5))
 (segment (start 102.616 121.936) (end 101.092 121.936) (width 1) (layer B.Cu) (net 5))
 (segment (start 116.586 125.492) (end 116.586 125.746) (width 1) (layer B.Cu) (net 5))
 (segment (start 111.506 128.032) (end 109.728 129.81) (width 1) (layer B.Cu) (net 5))
 (segment (start 114.3 128.032) (end 111.506 128.032) (width 1) (layer B.Cu) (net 5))
 (segment (start 116.586 125.746) (end 114.3 128.032) (width 1) (layer B.Cu) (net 5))
 (segment (start 103.632 122.952) (end 102.616 121.936) (width 1) (layer B.Cu) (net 5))
 (segment (start 106.172 122.952) (end 103.632 122.952) (width 1) (layer B.Cu) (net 5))
 (segment (start 124.206 130.064) (end 126.492 130.064) (width 1) (layer B.Cu) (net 20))
 (segment (start 129.286 127.27) (end 130.81 127.27) (width 1) (layer B.Cu) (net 20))
 (segment (start 126.492 130.064) (end 129.286 127.27) (width 1) (layer B.Cu) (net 20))
 (segment (start 140.97 107.712) (end 140.97 106.442) (width 1) (layer B.Cu) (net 16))
 (segment (start 133.35 104.918) (end 133.35 106.696) (width 1) (layer B.Cu) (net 16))
 (segment (start 134.112 104.156) (end 133.35 104.918) (width 1) (layer B.Cu) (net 16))
 (segment (start 138.684 104.156) (end 134.112 104.156) (width 1) (layer B.Cu) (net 16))
 (segment (start 140.97 106.442) (end 138.684 104.156) (width 1) (layer B.Cu) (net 16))
 (segment (start 130.81 112.03) (end 130.81 109.236) (width 1) (layer B.Cu) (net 16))
 (segment (start 130.81 109.236) (end 133.35 106.696) (width 1) (layer B.Cu) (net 16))
 (segment (start 153.162 133.62) (end 153.162 128.794) (width 1) (layer B.Cu) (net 7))
 (segment (start 152.4 128.032) (end 151.13 128.032) (width 1) (layer B.Cu) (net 7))
 (segment (start 153.162 128.794) (end 152.4 128.032) (width 1) (layer B.Cu) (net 7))
 (segment (start 125.73 138.7) (end 142.748 138.7) (width 1) (layer B.Cu) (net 8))
 (segment (start 116.586 133.112) (end 122.174 138.7) (width 1) (layer B.Cu) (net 8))
 (segment (start 125.73 138.7) (end 122.174 138.7) (width 1) (layer B.Cu) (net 8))
 (segment (start 144.526 136.922) (end 144.526 133.62) (width 1) (layer B.Cu) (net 8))
 (segment (start 142.748 138.7) (end 144.526 136.922) (width 1) (layer B.Cu) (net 8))
 (segment (start 124.206 133.112) (end 127.508 133.112) (width 1) (layer B.Cu) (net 22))
 (segment (start 128.27 132.35) (end 130.81 132.35) (width 1) (layer B.Cu) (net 22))
 (segment (start 127.508 133.112) (end 128.27 132.35) (width 1) (layer B.Cu) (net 22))
 (segment (start 154.686 109.49) (end 154.686 114.062) (width 1) (layer B.Cu) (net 12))
 (segment (start 158.496 117.872) (end 158.496 119.396) (width 1) (layer B.Cu) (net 12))
 (segment (start 154.686 114.062) (end 158.496 117.872) (width 1) (layer B.Cu) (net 12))
 (segment (start 101.092 123.968) (end 102.108 123.968) (width 1) (layer B.Cu) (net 6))
 (segment (start 102.108 123.968) (end 103.124 124.984) (width 1) (layer B.Cu) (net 6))
 (segment (start 112.776 132.858) (end 108.966 132.858) (width 1) (layer B.Cu) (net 6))
 (segment (start 108.966 132.858) (end 106.172 130.064) (width 1) (layer B.Cu) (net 6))
 (segment (start 116.586 130.064) (end 113.792 130.064) (width 1) (layer B.Cu) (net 6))
 (segment (start 113.792 130.064) (end 112.776 131.08) (width 1) (layer B.Cu) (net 6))
 (segment (start 112.776 131.08) (end 112.776 132.858) (width 1) (layer B.Cu) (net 6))
 (segment (start 103.124 124.984) (end 104.902 124.984) (width 1) (layer B.Cu) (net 6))
 (segment (start 104.902 124.984) (end 106.172 126.254) (width 1) (layer B.Cu) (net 6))
 (segment (start 106.172 130.064) (end 106.172 126.254) (width 1) (layer B.Cu) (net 6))
 (segment (start 124.46 113.3) (end 121.92 113.3) (width 1) (layer B.Cu) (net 4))
 (segment (start 120.65 112.03) (end 118.11 112.03) (width 1) (layer B.Cu) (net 4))
 (segment (start 121.92 113.3) (end 120.65 112.03) (width 1) (layer B.Cu) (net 4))
 (segment (start 130.81 119.65) (end 128.778 119.65) (width 1) (layer B.Cu) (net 4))
 (segment (start 126.492 113.3) (end 124.46 113.3) (width 1) (layer B.Cu) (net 4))
 (segment (start 127.508 114.316) (end 126.492 113.3) (width 1) (layer B.Cu) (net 4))
 (segment (start 127.508 118.38) (end 127.508 114.316) (width 1) (layer B.Cu) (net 4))
 (segment (start 128.778 119.65) (end 127.508 118.38) (width 1) (layer B.Cu) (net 4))
 (segment (start 124.206 125.492) (end 127.508 125.492) (width 1) (layer B.Cu) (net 19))
 (segment (start 128.27 124.73) (end 130.81 124.73) (width 1) (layer B.Cu) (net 19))
 (segment (start 127.508 125.492) (end 128.27 124.73) (width 1) (layer B.Cu) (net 19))
 (segment (start 138.43 119.65) (end 140.97 119.65) (width 1) (layer B.Cu) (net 17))
 (segment (start 148.844 113.554) (end 149.606 112.792) (width 1) (layer B.Cu) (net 17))
 (segment (start 148.844 121.936) (end 148.844 113.554) (width 1) (layer B.Cu) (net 17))
 (segment (start 147.828 122.952) (end 148.844 121.936) (width 1) (layer B.Cu) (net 17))
 (segment (start 144.272 122.952) (end 147.828 122.952) (width 1) (layer B.Cu) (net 17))
 (segment (start 140.97 119.65) (end 144.272 122.952) (width 1) (layer B.Cu) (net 17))
 (segment (start 144.018 116.348) (end 143.256 116.348) (width 1) (layer B.Cu) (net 18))
 (segment (start 141.478 114.57) (end 138.43 114.57) (width 1) (layer B.Cu) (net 18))
 (segment (start 143.256 116.348) (end 141.478 114.57) (width 1) (layer B.Cu) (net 18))
 (segment (start 118.11 120.92) (end 123.444 120.92) (width 1) (layer B.Cu) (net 3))
 (segment (start 123.444 120.92) (end 124.46 119.904) (width 1) (layer B.Cu) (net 3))
 (segment (start 130.81 122.19) (end 126.746 122.19) (width 1) (layer B.Cu) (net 3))
 (segment (start 124.46 119.904) (end 124.46 118.38) (width 1) (layer B.Cu) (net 3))
 (segment (start 126.746 122.19) (end 124.46 119.904) (width 1) (layer B.Cu) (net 3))
 (segment (start 138.43 132.35) (end 139.446 132.35) (width 1) (layer B.Cu) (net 21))
 (segment (start 143.51 128.286) (end 143.51 128.032) (width 1) (layer B.Cu) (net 21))
 (segment (start 139.446 132.35) (end 143.51 128.286) (width 1) (layer B.Cu) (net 21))
 (segment (start 152.4 106.95) (end 152.146 106.95) (width 1) (layer B.Cu) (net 1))
 (segment (start 152.146 106.95) (end 147.828 102.632) (width 1) (layer B.Cu) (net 1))
 (segment (start 111.76 111.776) (end 111.76 113.554) (width 1) (layer B.Cu) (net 1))
 (segment (start 114.3 109.236) (end 111.76 111.776) (width 1) (layer B.Cu) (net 1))
 (segment (start 124.968 109.236) (end 114.3 109.236) (width 1) (layer B.Cu) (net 1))
 (segment (start 131.572 102.632) (end 124.968 109.236) (width 1) (layer B.Cu) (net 1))
 (segment (start 147.828 102.632) (end 131.572 102.632) (width 1) (layer B.Cu) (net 1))
 (segment (start 101.092 126.508) (end 101.092 127.524) (width 1) (layer B.Cu) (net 1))
 (segment (start 160.274 106.95) (end 154.686 106.95) (width 1) (layer B.Cu) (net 1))
 (segment (start 162.56 109.236) (end 160.274 106.95) (width 1) (layer B.Cu) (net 1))
 (segment (start 162.56 134.128) (end 162.56 109.236) (width 1) (layer B.Cu) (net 1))
 (segment (start 155.956 140.732) (end 162.56 134.128) (width 1) (layer B.Cu) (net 1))
 (segment (start 114.3 140.732) (end 155.956 140.732) (width 1) (layer B.Cu) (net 1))
 (segment (start 101.092 127.524) (end 114.3 140.732) (width 1) (layer B.Cu) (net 1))
 (segment (start 148.59 107.712) (end 151.384 107.712) (width 1) (layer B.Cu) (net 1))
 (segment (start 152.4 106.95) (end 154.686 106.95) (width 1) (layer B.Cu) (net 1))
 (segment (start 151.384 107.712) (end 152.146 106.95) (width 1) (layer B.Cu) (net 1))
 (segment (start 138.43 112.03) (end 141.478 112.03) (width 1) (layer B.Cu) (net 1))
 (segment (start 145.796 107.712) (end 148.59 107.712) (width 1) (layer B.Cu) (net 1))
 (segment (start 141.478 112.03) (end 145.796 107.712) (width 1) (layer B.Cu) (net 1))
 (segment (start 106.172 118.634) (end 106.172 114.316) (width 1) (layer B.Cu) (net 1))
 (segment (start 107.696 112.792) (end 110.998 112.792) (width 1) (layer B.Cu) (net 1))
 (segment (start 110.998 112.792) (end 111.76 113.554) (width 1) (layer B.Cu) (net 1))
 (segment (start 106.172 114.316) (end 107.696 112.792) (width 1) (layer B.Cu) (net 1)))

